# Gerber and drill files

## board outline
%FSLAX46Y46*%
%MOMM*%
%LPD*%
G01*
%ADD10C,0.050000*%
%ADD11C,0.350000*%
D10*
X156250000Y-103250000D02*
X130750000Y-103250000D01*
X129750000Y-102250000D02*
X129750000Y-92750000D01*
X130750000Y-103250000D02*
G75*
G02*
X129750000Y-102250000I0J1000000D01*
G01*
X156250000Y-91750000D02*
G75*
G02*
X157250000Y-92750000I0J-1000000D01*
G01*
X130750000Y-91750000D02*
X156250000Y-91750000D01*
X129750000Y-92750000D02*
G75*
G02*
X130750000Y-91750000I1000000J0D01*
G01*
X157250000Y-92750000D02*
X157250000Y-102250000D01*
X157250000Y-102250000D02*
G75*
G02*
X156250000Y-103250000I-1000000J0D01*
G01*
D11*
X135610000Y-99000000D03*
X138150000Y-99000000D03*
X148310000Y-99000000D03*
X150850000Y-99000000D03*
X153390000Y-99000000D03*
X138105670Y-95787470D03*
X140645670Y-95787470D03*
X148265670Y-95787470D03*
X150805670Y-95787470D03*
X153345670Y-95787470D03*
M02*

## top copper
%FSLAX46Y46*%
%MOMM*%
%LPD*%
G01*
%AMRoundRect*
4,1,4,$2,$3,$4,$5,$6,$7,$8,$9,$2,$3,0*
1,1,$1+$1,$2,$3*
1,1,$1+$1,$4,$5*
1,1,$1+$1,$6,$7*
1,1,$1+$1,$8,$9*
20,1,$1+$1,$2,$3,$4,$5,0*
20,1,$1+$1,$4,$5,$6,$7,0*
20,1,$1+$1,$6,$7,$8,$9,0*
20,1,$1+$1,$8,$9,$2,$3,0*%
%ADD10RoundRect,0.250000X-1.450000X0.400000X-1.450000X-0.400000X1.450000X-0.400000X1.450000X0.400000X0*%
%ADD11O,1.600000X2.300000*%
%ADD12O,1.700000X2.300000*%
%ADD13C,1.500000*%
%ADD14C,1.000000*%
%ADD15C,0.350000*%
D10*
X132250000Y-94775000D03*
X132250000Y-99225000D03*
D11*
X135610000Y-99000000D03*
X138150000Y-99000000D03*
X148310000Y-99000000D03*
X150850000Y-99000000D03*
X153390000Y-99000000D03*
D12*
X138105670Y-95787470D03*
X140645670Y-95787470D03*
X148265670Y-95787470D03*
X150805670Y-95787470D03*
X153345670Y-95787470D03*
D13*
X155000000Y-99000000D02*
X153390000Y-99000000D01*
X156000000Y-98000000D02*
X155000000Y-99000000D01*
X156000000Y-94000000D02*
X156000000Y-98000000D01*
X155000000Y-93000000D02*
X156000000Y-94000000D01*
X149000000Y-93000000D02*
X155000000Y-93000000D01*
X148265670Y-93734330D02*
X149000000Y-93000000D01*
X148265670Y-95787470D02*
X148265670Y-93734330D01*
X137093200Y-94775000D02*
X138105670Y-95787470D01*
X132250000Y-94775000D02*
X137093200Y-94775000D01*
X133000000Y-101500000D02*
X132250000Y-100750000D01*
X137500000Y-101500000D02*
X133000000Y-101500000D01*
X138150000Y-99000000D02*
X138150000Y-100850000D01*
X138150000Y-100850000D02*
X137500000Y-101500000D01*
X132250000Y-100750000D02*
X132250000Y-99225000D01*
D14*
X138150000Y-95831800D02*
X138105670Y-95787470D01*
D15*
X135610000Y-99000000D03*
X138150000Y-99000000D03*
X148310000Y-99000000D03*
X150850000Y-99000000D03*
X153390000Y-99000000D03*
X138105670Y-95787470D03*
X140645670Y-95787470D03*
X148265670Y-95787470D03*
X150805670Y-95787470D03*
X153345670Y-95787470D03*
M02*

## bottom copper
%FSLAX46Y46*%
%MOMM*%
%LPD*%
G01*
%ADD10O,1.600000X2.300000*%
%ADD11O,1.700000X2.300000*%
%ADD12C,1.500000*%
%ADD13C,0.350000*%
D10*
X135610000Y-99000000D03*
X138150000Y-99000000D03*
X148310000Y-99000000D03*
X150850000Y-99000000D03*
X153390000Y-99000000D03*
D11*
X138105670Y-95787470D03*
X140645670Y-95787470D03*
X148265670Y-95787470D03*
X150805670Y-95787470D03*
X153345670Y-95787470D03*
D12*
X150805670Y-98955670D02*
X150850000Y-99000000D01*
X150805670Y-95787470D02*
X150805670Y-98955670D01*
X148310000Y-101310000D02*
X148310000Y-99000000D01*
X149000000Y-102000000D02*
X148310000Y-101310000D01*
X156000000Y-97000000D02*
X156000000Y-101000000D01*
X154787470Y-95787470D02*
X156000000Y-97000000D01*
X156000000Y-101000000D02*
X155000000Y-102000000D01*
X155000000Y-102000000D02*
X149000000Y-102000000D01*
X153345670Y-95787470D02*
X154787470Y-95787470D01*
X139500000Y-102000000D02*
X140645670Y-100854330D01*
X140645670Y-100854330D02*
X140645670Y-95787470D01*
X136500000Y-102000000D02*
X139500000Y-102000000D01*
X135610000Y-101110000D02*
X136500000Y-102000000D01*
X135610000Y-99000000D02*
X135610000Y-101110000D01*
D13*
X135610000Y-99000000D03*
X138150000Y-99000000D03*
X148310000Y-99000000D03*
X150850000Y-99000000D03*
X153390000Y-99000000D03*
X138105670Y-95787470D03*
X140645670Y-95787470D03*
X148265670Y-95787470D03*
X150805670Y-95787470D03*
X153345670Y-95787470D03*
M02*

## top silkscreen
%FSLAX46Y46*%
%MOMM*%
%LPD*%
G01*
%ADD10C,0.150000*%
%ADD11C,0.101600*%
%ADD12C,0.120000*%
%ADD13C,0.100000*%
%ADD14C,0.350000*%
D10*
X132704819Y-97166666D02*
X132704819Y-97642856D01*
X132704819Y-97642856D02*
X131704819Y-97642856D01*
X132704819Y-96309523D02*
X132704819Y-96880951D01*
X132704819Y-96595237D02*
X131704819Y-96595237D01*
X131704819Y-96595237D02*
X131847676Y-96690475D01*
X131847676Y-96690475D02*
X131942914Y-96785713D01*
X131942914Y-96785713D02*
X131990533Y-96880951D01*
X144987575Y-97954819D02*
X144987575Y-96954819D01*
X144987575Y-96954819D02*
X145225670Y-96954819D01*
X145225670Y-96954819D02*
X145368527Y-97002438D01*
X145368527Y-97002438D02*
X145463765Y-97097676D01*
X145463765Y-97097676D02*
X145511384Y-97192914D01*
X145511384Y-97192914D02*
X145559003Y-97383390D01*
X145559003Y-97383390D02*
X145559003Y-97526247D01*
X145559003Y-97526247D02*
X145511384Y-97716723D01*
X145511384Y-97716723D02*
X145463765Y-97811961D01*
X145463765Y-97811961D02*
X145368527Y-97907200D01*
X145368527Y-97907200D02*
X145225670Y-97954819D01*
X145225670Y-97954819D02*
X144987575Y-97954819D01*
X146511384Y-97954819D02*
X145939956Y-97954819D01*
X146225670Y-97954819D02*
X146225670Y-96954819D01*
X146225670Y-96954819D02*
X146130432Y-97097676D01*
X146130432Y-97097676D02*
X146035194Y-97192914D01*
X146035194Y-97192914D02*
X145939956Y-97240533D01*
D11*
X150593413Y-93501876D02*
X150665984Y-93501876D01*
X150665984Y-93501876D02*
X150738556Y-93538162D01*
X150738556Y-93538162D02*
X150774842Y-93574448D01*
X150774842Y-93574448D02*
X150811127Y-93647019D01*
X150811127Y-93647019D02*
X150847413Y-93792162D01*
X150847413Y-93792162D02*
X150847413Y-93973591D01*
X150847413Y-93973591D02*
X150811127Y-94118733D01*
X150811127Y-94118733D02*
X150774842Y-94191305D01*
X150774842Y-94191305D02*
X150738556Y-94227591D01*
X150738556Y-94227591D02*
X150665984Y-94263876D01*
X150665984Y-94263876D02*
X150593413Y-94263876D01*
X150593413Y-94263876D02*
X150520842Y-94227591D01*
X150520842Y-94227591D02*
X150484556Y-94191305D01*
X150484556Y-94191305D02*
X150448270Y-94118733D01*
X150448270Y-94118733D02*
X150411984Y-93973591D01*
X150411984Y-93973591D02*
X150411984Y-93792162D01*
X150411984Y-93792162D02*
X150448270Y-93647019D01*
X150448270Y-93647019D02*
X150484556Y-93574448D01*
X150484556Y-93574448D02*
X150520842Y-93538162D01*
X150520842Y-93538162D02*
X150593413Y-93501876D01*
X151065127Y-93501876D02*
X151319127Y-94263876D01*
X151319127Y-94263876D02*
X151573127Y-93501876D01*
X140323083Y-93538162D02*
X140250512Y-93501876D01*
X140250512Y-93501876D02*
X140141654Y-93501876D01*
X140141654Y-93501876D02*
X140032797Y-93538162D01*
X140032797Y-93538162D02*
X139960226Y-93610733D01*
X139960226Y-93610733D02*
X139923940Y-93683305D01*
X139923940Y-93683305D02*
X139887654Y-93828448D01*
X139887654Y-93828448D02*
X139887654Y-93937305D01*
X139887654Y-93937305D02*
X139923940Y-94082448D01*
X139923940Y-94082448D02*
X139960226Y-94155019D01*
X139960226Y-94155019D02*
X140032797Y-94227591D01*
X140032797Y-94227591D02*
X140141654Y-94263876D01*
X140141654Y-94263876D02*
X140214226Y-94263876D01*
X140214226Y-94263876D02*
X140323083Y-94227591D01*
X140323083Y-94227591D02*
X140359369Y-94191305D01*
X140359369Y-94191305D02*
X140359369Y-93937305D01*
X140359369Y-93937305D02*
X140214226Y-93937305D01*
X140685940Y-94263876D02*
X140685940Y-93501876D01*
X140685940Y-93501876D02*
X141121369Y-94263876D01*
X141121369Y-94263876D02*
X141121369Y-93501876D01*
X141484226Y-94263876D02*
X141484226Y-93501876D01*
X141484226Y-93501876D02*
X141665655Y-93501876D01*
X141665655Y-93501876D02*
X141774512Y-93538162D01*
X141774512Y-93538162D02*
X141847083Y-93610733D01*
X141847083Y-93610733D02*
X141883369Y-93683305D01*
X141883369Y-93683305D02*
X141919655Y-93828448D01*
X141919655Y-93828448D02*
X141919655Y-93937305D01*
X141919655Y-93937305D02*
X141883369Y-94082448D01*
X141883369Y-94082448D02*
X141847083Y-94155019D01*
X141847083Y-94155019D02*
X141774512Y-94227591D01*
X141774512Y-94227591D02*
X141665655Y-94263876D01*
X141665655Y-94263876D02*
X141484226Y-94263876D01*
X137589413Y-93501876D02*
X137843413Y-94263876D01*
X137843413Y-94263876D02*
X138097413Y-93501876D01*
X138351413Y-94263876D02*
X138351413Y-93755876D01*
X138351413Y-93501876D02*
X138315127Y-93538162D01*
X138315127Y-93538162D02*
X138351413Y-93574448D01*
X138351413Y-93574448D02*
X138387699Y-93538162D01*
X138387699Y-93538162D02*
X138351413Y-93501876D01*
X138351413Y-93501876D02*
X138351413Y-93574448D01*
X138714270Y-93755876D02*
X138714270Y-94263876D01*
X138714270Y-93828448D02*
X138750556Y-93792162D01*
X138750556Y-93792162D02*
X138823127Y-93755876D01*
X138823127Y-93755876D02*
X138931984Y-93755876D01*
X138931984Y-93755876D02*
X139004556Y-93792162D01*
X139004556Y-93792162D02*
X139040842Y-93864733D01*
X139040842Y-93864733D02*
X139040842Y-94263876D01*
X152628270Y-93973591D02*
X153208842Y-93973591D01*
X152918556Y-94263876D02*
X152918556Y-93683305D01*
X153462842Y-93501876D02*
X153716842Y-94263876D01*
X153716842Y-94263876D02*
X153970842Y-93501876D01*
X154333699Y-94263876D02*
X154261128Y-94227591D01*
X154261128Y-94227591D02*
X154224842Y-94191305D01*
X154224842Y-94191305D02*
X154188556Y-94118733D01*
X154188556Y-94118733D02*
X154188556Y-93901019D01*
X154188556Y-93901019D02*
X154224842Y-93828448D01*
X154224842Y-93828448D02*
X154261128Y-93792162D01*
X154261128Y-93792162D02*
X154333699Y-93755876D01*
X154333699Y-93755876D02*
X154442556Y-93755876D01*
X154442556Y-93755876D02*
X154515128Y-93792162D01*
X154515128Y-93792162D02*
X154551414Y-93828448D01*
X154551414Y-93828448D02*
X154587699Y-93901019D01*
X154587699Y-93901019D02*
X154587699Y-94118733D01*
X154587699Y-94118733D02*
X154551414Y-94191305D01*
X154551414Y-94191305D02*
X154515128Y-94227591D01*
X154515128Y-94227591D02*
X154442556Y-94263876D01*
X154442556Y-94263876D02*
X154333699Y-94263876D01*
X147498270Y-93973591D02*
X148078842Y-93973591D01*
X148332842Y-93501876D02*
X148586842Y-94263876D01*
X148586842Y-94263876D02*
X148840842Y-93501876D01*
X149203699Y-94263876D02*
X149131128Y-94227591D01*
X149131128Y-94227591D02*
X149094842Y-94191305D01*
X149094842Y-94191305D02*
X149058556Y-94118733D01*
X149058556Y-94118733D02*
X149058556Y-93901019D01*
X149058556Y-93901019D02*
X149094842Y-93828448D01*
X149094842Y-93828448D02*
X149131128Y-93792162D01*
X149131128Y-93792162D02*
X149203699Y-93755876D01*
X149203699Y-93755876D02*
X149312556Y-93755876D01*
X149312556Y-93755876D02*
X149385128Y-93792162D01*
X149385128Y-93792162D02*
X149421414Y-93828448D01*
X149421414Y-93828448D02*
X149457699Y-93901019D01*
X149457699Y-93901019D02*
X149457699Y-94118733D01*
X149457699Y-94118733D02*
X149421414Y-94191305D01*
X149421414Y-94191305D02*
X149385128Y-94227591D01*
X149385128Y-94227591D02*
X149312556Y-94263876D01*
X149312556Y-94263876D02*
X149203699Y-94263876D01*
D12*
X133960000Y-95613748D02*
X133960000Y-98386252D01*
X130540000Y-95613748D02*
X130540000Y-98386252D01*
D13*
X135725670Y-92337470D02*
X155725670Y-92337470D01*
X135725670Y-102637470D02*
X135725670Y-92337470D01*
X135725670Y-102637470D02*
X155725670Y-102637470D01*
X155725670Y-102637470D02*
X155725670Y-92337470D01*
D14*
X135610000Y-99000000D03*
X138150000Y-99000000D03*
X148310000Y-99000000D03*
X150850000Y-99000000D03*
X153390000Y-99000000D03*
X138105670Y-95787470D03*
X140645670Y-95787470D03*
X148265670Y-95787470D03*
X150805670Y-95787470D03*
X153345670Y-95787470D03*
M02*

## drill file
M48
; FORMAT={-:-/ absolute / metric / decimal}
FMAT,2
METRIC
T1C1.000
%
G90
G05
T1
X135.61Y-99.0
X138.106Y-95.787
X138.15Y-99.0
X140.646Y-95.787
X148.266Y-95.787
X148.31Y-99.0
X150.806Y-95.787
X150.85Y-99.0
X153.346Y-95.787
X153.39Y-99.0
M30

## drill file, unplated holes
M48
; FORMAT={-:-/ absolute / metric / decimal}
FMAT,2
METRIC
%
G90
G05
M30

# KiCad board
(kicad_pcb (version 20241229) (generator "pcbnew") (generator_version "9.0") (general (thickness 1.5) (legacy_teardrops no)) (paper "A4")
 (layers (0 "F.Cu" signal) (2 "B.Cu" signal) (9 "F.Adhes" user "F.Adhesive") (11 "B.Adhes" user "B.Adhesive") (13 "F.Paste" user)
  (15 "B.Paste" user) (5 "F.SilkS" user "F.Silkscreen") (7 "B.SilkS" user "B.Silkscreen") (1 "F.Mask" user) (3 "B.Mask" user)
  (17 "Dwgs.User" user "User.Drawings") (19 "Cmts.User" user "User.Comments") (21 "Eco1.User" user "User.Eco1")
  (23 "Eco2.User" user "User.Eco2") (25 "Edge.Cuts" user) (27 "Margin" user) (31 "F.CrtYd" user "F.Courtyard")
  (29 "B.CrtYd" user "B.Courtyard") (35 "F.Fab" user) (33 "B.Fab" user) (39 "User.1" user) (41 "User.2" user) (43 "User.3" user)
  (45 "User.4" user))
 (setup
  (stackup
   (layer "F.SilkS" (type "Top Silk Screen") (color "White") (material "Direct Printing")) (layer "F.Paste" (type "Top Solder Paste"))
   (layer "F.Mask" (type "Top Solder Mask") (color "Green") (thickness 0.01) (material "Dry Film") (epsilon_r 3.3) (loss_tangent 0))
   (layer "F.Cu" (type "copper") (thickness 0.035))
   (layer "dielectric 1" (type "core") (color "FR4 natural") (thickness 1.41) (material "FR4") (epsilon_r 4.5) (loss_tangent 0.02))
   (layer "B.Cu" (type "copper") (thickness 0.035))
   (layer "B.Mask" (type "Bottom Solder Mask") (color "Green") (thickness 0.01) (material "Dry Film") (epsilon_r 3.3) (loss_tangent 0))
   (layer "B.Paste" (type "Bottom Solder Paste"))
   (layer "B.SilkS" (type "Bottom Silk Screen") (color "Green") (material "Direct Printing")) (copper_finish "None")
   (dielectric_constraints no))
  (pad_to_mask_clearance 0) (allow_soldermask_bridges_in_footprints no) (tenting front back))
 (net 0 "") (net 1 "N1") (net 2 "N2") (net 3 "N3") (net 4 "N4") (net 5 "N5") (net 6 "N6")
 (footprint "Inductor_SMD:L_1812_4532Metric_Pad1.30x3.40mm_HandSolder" (layer "F.Cu") (at 132.25 97 -90)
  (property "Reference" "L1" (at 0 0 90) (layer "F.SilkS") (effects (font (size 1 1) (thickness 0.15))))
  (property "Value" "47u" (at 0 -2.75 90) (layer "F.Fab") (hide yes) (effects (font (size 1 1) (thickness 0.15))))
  (fp_line (start -1.386252 1.71) (end 1.386252 1.71) (stroke (width 0.12) (type solid)) (layer "F.SilkS"))
  (fp_line (start -1.386252 -1.71) (end 1.386252 -1.71) (stroke (width 0.12) (type solid)) (layer "F.SilkS"))
  (pad "1" smd roundrect (at -2.225 0 270) (size 1.3 3.4) (layers "F.Cu" "F.Mask" "F.Paste") (roundrect_rratio 0.192308) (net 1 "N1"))
  (pad "2" smd roundrect (at 2.225 0 270) (size 1.3 3.4) (layers "F.Cu" "F.Mask" "F.Paste") (roundrect_rratio 0.192308) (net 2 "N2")))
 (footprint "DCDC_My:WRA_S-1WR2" (layer "F.Cu") (at 144.5 99)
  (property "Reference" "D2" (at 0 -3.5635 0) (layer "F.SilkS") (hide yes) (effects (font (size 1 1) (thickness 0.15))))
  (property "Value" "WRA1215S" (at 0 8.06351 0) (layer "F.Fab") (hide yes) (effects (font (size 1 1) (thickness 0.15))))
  (pad "1" thru_hole oval (at -8.89 0) (size 1.6 2.3) (drill 1) (layers "*.Cu" "*.Mask") (remove_unused_layers no) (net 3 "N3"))
  (pad "2" thru_hole oval (at -6.35 0) (size 1.6 2.3) (drill 1) (layers "*.Cu" "*.Mask") (remove_unused_layers no) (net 2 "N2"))
  (pad "6" thru_hole oval (at 3.81 0) (size 1.6 2.3) (drill 1) (layers "*.Cu" "*.Mask") (remove_unused_layers no) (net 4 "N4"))
  (pad "7" thru_hole oval (at 6.35 0) (size 1.6 2.3) (drill 1) (layers "*.Cu" "*.Mask") (remove_unused_layers no) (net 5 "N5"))
  (pad "8" thru_hole oval (at 8.89 0) (size 1.6 2.3) (drill 1) (layers "*.Cu" "*.Mask") (remove_unused_layers no) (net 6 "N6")))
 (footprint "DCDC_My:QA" (layer "F.Cu") (at 145.75 97.5)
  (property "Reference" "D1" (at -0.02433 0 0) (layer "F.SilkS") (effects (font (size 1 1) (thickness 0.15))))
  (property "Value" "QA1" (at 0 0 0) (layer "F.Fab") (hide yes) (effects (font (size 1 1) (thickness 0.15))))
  (fp_line (start -10.02433 -5.16253) (end 9.97567 -5.16253) (stroke (width 0.1) (type solid)) (layer "F.SilkS"))
  (fp_line (start -10.02433 5.13747) (end -10.02433 -5.16253) (stroke (width 0.1) (type solid)) (layer "F.SilkS"))
  (fp_line (start -10.02433 5.13747) (end 9.97567 5.13747) (stroke (width 0.1) (type solid)) (layer "F.SilkS"))
  (fp_line (start 9.97567 5.13747) (end 9.97567 -5.16253) (stroke (width 0.1) (type solid)) (layer "F.SilkS"))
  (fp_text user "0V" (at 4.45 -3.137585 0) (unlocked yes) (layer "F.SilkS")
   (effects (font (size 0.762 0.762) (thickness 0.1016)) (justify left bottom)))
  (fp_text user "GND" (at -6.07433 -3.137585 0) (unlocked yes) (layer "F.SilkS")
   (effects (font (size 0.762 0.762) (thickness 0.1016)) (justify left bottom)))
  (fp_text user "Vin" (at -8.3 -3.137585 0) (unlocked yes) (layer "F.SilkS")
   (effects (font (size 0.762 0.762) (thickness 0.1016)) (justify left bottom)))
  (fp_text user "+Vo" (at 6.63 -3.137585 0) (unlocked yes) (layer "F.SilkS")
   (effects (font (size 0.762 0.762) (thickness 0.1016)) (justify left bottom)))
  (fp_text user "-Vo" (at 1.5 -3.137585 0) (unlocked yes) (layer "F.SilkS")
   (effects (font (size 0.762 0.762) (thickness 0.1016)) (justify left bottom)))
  (pad "1" thru_hole oval (at -7.64433 -1.71253) (size 1.7 2.3) (drill 1) (layers "*.Cu" "*.Mask") (remove_unused_layers no) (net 1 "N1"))
  (pad "2" thru_hole oval (at -5.10433 -1.71253 180) (size 1.7 2.3) (drill 1) (layers "*.Cu" "*.Mask") (remove_unused_layers no)
   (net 3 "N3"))
  (pad "5" thru_hole oval (at 2.51567 -1.71253 180) (size 1.7 2.3) (drill 1) (layers "*.Cu" "*.Mask") (remove_unused_layers no) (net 6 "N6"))
  (pad "6" thru_hole oval (at 5.05567 -1.71253 180) (size 1.7 2.3) (drill 1) (layers "*.Cu" "*.Mask") (remove_unused_layers no) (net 5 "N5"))
  (pad "7" thru_hole oval (at 7.59567 -1.71253) (size 1.7 2.3) (drill 1) (layers "*.Cu" "*.Mask") (remove_unused_layers no) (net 4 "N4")))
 (gr_line (start 156.25 103.25) (end 130.75 103.25) (stroke (width 0.05) (type default)) (layer "Edge.Cuts"))
 (gr_line (start 129.75 102.25) (end 129.75 92.75) (stroke (width 0.05) (type default)) (layer "Edge.Cuts"))
 (gr_arc (start 130.75 103.25) (mid 130.042893 102.957107) (end 129.75 102.25) (stroke (width 0.05) (type default)) (layer "Edge.Cuts"))
 (gr_arc (start 156.25 91.75) (mid 156.957107 92.042893) (end 157.25 92.75) (stroke (width 0.05) (type default)) (layer "Edge.Cuts"))
 (gr_line (start 130.75 91.75) (end 156.25 91.75) (stroke (width 0.05) (type default)) (layer "Edge.Cuts"))
 (gr_arc (start 129.75 92.75) (mid 130.042893 92.042893) (end 130.75 91.75) (stroke (width 0.05) (type default)) (layer "Edge.Cuts"))
 (gr_line (start 157.25 92.75) (end 157.25 102.25) (stroke (width 0.05) (type default)) (layer "Edge.Cuts"))
 (gr_arc (start 157.25 102.25) (mid 156.957107 102.957107) (end 156.25 103.25) (stroke (width 0.05) (type default)) (layer "Edge.Cuts"))
 (segment (start 138.15 95.8318) (end 138.10567 95.78747) (width 1) (layer "F.Cu") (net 1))
 (segment (start 137.0932 94.775) (end 138.10567 95.78747) (width 1.5) (layer "F.Cu") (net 1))
 (segment (start 132.25 94.775) (end 137.0932 94.775) (width 1.5) (layer "F.Cu") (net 1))
 (segment (start 139.5 102) (end 140.64567 100.85433) (width 1.5) (layer "B.Cu") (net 3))
 (segment (start 140.64567 100.85433) (end 140.64567 95.78747) (width 1.5) (layer "B.Cu") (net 3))
 (segment (start 135.61 101.11) (end 136.5 102) (width 1.5) (layer "B.Cu") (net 3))
 (segment (start 135.61 99) (end 135.61 101.11) (width 1.5) (layer "B.Cu") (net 3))
 (segment (start 136.5 102) (end 139.5 102) (width 1.5) (layer "B.Cu") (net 3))
 (segment (start 150.80567 98.95567) (end 150.85 99) (width 1.5) (layer "B.Cu") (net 5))
 (segment (start 150.80567 95.78747) (end 150.80567 98.95567) (width 1.5) (layer "B.Cu") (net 5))
 (segment (start 155 102) (end 149 102) (width 1.5) (layer "B.Cu") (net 4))
 (segment (start 156 97) (end 156 101) (width 1.5) (layer "B.Cu") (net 4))
 (segment (start 154.78747 95.78747) (end 156 97) (width 1.5) (layer "B.Cu") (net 4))
 (segment (start 148.31 101.31) (end 148.31 99) (width 1.5) (layer "B.Cu") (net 4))
 (segment (start 156 101) (end 155 102) (width 1.5) (layer "B.Cu") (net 4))
 (segment (start 149 102) (end 148.31 101.31) (width 1.5) (layer "B.Cu") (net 4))
 (segment (start 153.34567 95.78747) (end 154.78747 95.78747) (width 1.5) (layer "B.Cu") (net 4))
 (segment (start 156 98) (end 155 99) (width 1.5) (layer "F.Cu") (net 6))
 (segment (start 148.26567 93.73433) (end 149 93) (width 1.5) (layer "F.Cu") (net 6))
 (segment (start 149 93) (end 155 93) (width 1.5) (layer "F.Cu") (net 6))
 (segment (start 148.26567 95.78747) (end 148.26567 93.73433) (width 1.5) (layer "F.Cu") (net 6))
 (segment (start 155 93) (end 156 94) (width 1.5) (layer "F.Cu") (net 6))
 (segment (start 155 99) (end 153.39 99) (width 1.5) (layer "F.Cu") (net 6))
 (segment (start 156 94) (end 156 98) (width 1.5) (layer "F.Cu") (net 6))
 (segment (start 132.25 100.75) (end 132.25 99.225) (width 1.5) (layer "F.Cu") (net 2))
 (segment (start 137.5 101.5) (end 133 101.5) (width 1.5) (layer "F.Cu") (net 2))
 (segment (start 138.15 99) (end 138.15 100.85) (width 1.5) (layer "F.Cu") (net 2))
 (segment (start 138.15 100.85) (end 137.5 101.5) (width 1.5) (layer "F.Cu") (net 2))
 (segment (start 133 101.5) (end 132.25 100.75) (width 1.5) (layer "F.Cu") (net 2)))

